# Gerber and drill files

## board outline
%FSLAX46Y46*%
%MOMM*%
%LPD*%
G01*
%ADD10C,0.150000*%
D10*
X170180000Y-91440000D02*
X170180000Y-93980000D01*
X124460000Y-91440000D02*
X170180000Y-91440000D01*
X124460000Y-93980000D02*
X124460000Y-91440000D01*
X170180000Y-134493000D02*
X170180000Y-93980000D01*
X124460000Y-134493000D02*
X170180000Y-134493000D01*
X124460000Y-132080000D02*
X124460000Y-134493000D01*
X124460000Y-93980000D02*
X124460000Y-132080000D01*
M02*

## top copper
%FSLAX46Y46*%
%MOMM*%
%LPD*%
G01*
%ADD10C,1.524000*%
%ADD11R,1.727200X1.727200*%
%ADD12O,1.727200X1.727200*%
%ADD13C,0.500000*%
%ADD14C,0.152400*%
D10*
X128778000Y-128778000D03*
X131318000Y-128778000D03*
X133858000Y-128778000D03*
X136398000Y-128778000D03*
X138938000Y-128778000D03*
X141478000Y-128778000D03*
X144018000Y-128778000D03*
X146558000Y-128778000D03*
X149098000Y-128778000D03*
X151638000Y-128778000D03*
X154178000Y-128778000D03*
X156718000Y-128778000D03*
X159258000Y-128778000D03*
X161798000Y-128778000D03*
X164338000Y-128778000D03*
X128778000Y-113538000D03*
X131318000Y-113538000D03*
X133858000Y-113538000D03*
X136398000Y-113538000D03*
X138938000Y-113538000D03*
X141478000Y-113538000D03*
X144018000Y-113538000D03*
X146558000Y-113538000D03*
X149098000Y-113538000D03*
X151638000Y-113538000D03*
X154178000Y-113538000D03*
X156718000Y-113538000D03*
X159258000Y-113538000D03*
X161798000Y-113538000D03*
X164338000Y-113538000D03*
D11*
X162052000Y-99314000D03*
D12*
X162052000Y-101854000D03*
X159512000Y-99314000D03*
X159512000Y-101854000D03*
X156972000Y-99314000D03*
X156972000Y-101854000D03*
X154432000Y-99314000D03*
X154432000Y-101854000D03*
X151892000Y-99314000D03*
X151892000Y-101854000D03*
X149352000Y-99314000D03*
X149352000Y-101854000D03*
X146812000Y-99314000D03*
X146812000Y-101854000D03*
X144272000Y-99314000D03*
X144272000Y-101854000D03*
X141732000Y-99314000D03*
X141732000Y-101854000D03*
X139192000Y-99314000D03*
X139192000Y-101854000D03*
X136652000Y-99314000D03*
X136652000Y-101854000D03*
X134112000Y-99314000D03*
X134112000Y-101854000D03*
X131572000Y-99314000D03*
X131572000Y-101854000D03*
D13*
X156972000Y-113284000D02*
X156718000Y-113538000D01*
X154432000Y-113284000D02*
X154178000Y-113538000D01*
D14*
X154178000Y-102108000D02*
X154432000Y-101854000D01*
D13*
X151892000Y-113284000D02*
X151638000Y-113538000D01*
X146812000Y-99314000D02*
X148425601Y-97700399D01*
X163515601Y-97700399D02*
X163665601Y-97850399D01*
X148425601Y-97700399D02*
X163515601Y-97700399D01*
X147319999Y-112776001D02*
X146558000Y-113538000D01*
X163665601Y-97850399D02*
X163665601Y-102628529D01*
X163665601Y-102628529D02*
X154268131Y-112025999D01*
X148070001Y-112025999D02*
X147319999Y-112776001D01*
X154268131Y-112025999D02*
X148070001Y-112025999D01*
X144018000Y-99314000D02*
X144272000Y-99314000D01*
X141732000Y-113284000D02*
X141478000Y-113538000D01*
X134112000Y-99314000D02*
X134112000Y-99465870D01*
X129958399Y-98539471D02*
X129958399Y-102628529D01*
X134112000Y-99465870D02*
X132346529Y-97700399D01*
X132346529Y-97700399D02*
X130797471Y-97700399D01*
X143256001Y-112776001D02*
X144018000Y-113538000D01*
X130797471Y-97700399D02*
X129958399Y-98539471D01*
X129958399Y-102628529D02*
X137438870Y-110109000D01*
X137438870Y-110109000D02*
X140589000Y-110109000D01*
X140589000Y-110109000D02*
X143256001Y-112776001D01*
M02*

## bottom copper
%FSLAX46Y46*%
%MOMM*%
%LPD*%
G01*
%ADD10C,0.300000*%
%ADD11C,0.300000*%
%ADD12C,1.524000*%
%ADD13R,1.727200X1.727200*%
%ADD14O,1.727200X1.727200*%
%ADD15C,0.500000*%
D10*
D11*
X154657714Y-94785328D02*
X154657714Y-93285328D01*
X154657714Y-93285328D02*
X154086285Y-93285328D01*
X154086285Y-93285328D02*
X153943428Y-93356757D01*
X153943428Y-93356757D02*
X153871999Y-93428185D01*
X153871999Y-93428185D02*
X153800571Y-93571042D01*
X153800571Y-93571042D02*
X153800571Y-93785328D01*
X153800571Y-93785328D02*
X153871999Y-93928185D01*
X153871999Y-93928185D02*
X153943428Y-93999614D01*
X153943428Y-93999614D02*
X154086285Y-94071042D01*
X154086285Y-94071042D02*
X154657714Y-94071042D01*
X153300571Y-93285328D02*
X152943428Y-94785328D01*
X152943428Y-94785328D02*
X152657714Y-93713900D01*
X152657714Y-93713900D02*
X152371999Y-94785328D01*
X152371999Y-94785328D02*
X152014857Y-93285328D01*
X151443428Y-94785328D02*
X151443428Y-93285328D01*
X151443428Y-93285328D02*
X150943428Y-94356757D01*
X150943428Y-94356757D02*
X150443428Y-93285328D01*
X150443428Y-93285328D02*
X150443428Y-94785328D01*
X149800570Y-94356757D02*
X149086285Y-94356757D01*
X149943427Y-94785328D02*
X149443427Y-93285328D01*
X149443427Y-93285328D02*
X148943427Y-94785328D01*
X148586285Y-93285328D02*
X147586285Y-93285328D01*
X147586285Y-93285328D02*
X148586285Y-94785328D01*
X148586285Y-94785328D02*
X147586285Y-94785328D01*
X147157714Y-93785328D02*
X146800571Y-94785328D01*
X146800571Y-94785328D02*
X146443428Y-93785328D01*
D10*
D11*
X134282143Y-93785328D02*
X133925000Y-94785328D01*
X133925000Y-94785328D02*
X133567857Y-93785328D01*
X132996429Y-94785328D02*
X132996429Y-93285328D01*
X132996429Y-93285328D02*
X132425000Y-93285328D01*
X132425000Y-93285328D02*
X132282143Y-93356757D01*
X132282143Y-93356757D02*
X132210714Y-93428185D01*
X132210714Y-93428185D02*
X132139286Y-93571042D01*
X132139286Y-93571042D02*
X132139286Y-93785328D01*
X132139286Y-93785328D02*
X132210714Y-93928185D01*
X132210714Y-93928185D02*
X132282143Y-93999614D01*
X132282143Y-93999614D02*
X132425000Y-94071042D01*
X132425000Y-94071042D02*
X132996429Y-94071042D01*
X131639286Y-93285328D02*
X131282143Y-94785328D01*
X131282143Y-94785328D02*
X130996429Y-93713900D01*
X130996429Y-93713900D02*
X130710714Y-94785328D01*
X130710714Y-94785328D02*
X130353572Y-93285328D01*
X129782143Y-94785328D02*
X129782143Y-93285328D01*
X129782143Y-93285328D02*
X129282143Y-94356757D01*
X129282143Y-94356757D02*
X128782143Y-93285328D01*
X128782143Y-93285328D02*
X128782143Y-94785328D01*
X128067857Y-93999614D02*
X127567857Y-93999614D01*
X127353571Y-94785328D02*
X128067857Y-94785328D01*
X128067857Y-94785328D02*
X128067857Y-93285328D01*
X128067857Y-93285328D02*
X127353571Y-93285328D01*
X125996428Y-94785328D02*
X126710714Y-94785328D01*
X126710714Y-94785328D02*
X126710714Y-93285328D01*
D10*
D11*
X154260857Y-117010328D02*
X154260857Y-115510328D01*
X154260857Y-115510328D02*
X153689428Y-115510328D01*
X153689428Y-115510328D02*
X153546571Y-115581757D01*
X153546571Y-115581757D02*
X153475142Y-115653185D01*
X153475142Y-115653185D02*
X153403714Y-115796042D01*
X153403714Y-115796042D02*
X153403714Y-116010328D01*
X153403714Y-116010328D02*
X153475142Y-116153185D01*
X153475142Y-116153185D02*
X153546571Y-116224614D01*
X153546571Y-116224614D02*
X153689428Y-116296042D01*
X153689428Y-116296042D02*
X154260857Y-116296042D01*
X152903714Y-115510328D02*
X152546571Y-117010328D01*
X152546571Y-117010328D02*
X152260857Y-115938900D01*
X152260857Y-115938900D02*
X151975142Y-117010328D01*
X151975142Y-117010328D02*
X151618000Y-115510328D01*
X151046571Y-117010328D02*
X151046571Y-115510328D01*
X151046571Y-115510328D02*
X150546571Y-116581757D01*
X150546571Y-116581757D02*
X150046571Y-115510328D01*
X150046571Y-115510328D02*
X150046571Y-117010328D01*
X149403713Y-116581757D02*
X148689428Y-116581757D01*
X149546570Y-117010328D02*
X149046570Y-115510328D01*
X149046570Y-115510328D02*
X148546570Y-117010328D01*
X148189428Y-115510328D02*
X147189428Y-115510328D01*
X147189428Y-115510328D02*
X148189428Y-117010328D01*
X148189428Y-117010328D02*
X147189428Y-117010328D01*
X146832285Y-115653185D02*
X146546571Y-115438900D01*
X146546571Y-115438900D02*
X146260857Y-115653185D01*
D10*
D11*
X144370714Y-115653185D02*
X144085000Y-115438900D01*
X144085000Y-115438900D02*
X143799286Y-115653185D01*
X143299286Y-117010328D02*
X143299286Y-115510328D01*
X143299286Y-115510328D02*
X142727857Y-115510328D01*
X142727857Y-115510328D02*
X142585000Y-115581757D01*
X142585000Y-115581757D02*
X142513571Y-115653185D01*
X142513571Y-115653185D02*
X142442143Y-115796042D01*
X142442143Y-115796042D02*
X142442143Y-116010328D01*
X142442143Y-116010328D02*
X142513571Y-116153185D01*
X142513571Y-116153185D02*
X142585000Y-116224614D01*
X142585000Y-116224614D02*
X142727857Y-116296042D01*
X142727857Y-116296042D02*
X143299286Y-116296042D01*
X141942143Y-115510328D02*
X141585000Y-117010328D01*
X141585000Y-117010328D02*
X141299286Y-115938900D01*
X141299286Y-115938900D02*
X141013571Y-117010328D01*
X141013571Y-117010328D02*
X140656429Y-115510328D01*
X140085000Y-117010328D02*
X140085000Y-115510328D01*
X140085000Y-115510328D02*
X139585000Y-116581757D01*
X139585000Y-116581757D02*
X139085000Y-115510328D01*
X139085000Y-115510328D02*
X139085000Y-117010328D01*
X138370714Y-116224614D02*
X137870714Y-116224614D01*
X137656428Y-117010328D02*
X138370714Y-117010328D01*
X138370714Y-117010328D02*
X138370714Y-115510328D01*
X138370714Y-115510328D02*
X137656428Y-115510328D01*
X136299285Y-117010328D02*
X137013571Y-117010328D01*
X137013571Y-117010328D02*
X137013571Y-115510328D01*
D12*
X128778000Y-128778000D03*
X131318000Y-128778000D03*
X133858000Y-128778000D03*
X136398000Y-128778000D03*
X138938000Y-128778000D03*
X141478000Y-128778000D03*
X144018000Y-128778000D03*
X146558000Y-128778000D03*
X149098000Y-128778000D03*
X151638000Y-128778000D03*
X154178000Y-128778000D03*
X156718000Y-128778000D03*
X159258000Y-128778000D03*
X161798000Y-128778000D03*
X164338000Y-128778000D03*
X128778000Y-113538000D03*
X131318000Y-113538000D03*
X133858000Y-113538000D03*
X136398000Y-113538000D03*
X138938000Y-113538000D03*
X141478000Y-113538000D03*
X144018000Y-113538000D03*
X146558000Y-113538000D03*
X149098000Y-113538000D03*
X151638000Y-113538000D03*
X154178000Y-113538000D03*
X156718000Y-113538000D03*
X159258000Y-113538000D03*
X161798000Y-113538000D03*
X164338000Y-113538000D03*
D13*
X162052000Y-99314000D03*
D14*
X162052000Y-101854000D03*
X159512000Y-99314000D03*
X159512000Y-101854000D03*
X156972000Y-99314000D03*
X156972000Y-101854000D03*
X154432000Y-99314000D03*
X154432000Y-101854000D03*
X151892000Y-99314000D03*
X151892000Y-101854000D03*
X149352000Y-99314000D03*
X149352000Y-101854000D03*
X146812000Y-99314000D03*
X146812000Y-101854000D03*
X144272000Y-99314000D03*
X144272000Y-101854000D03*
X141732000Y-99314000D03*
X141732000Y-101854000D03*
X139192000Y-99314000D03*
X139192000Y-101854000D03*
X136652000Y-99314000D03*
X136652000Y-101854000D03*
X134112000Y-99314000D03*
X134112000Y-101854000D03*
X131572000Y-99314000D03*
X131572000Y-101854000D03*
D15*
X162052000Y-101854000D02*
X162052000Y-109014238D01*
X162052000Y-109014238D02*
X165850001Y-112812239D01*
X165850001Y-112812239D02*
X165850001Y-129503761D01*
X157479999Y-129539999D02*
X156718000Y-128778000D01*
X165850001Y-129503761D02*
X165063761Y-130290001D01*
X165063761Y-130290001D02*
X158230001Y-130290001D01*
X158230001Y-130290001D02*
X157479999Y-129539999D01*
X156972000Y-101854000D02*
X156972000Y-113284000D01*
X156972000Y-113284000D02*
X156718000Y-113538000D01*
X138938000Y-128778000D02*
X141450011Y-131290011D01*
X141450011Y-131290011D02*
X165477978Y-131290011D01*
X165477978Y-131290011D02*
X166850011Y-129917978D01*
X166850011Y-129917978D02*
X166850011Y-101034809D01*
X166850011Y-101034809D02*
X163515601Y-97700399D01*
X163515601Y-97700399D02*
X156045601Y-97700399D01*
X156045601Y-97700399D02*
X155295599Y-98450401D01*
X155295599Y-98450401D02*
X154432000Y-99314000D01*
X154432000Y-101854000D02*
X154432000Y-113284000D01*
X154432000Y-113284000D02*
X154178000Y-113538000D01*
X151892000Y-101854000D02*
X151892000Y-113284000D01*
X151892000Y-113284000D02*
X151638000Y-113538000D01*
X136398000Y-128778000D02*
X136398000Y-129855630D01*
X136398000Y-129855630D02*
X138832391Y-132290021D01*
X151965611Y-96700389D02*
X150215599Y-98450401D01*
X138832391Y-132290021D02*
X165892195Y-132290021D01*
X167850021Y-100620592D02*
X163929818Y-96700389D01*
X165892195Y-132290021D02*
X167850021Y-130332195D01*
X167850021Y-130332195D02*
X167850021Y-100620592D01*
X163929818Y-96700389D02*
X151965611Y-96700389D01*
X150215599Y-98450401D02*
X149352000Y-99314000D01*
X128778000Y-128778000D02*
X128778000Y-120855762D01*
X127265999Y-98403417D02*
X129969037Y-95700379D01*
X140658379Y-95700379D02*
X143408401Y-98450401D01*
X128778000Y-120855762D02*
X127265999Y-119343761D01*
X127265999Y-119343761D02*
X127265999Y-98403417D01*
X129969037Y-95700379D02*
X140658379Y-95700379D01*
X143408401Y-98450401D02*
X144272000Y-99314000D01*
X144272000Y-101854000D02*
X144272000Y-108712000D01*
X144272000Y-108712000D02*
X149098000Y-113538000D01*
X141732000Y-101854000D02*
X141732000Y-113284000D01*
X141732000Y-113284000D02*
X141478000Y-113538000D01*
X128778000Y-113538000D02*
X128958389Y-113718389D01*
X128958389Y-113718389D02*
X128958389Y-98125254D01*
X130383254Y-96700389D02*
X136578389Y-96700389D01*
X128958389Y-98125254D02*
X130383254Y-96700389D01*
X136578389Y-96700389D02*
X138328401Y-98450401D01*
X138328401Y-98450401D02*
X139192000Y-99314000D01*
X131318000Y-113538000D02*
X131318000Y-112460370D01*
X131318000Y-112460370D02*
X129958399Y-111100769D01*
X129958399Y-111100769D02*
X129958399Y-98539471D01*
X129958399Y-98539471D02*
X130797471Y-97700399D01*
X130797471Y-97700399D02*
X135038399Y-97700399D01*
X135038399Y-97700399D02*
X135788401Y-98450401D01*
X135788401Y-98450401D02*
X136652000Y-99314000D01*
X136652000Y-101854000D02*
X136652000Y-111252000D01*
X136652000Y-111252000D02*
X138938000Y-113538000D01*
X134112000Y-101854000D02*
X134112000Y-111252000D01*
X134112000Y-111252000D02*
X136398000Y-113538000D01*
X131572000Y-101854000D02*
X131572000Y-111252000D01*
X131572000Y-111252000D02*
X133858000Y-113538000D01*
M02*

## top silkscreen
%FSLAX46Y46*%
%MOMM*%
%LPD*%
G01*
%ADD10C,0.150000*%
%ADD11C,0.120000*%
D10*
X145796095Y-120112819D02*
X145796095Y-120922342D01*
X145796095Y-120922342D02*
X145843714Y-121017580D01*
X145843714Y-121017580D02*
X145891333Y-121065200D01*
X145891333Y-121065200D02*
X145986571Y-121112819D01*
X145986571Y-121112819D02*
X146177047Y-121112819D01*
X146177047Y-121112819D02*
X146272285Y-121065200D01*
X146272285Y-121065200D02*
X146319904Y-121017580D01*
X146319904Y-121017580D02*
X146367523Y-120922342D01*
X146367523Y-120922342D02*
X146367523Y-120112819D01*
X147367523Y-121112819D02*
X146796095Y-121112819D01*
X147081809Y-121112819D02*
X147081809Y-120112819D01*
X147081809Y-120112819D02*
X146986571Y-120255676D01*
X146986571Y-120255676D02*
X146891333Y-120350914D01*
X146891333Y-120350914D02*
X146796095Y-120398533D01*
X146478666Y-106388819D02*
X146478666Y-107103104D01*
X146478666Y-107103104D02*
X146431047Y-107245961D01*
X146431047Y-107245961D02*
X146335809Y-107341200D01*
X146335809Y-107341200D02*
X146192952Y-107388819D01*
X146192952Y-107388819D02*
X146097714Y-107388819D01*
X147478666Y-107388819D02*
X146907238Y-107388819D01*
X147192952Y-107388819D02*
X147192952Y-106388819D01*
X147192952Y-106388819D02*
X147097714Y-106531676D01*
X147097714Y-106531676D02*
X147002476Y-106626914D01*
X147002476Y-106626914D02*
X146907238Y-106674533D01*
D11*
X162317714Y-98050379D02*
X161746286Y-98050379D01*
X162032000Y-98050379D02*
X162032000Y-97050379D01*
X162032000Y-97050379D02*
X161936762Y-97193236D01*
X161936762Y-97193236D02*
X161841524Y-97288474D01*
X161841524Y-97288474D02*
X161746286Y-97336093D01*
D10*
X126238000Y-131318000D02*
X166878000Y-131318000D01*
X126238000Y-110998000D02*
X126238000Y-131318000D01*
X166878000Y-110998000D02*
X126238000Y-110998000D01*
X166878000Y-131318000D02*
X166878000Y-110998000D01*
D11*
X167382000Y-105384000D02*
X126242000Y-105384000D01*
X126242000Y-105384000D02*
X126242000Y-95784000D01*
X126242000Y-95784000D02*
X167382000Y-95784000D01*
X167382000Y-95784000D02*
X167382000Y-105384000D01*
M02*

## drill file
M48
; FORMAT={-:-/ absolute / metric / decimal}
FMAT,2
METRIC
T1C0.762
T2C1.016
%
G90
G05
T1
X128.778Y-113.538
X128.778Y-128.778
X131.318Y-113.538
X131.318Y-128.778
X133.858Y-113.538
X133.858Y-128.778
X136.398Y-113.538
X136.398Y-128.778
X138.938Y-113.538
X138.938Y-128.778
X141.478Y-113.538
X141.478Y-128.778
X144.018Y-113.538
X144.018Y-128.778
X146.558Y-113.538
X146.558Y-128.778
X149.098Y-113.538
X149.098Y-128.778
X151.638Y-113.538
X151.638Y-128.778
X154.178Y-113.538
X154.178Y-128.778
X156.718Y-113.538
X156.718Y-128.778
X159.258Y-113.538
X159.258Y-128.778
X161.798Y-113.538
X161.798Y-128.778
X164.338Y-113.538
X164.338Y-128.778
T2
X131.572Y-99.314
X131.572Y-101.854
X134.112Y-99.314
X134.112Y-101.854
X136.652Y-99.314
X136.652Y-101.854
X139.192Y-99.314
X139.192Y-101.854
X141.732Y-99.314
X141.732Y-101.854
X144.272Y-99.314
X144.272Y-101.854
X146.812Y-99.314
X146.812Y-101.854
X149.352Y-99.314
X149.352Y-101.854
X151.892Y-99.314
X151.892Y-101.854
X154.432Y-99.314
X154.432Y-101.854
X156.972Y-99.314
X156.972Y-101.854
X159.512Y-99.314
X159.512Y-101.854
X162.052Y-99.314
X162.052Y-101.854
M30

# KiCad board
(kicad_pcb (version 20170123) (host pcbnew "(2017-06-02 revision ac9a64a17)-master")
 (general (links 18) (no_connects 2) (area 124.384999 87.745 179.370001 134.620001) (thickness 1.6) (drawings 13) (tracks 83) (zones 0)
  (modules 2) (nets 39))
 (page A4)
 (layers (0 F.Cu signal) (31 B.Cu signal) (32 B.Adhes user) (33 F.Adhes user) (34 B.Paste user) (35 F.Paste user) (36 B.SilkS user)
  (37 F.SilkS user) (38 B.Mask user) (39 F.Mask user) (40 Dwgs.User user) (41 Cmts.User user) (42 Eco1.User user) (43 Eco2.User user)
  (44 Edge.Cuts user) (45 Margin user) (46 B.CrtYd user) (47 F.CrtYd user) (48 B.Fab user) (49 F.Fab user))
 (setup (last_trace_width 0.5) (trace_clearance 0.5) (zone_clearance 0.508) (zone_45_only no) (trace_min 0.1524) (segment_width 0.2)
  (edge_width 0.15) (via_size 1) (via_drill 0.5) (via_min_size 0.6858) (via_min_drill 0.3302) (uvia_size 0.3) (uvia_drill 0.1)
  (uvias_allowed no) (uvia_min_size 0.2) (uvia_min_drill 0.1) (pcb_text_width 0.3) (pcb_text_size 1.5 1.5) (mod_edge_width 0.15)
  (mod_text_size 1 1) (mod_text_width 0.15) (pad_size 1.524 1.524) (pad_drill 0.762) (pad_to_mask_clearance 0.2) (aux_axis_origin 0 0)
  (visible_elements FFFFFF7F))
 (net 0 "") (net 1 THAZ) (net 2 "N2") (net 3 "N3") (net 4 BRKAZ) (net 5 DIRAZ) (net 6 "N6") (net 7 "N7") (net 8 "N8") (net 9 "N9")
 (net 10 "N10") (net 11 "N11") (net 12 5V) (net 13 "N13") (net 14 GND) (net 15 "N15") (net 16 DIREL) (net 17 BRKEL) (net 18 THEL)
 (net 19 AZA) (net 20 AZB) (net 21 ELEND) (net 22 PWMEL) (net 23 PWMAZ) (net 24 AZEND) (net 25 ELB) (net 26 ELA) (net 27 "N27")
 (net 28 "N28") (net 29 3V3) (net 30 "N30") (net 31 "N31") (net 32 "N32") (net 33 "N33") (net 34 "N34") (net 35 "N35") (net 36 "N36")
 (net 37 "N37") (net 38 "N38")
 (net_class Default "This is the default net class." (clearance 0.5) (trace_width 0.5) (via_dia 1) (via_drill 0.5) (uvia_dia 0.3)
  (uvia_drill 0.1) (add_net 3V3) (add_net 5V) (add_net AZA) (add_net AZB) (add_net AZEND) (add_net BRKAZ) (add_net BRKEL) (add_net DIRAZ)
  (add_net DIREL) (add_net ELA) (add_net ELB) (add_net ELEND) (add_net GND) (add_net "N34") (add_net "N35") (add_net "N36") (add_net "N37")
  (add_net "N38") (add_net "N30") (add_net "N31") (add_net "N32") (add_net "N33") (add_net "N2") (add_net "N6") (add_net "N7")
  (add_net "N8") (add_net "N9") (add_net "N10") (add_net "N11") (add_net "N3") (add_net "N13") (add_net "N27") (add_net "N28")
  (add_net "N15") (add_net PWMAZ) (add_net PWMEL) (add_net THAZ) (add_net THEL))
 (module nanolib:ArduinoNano (layer F.Cu) (at 146.558 121.158 180)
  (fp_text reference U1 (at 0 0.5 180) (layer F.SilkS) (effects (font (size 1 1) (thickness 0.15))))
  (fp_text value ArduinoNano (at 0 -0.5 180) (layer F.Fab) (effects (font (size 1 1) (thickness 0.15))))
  (fp_line (start 20.32 -10.16) (end -20.32 -10.16) (layer F.SilkS) (width 0.15))
  (fp_line (start 20.32 10.16) (end 20.32 -10.16) (layer F.SilkS) (width 0.15))
  (fp_line (start -20.32 10.16) (end 20.32 10.16) (layer F.SilkS) (width 0.15))
  (fp_line (start -20.32 -10.16) (end -20.32 10.16) (layer F.SilkS) (width 0.15))
  (pad D13 thru_hole circle (at 17.78 -7.62 180) (size 1.524 1.524) (drill 0.762) (layers *.Cu *.Mask) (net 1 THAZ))
  (pad 3V3 thru_hole circle (at 15.24 -7.62 180) (size 1.524 1.524) (drill 0.762) (layers *.Cu *.Mask) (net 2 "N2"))
  (pad REF thru_hole circle (at 12.7 -7.62 180) (size 1.524 1.524) (drill 0.762) (layers *.Cu *.Mask) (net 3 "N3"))
  (pad A0 thru_hole circle (at 10.16 -7.62 180) (size 1.524 1.524) (drill 0.762) (layers *.Cu *.Mask) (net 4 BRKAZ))
  (pad A1 thru_hole circle (at 7.62 -7.62 180) (size 1.524 1.524) (drill 0.762) (layers *.Cu *.Mask) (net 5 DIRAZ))
  (pad A2 thru_hole circle (at 5.08 -7.62 180) (size 1.524 1.524) (drill 0.762) (layers *.Cu *.Mask) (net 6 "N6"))
  (pad A3 thru_hole circle (at 2.54 -7.62 180) (size 1.524 1.524) (drill 0.762) (layers *.Cu *.Mask) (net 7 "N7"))
  (pad A4 thru_hole circle (at 0 -7.62 180) (size 1.524 1.524) (drill 0.762) (layers *.Cu *.Mask) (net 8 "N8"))
  (pad A5 thru_hole circle (at -2.54 -7.62 180) (size 1.524 1.524) (drill 0.762) (layers *.Cu *.Mask) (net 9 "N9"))
  (pad A6 thru_hole circle (at -5.08 -7.62 180) (size 1.524 1.524) (drill 0.762) (layers *.Cu *.Mask) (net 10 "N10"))
  (pad A7 thru_hole circle (at -7.62 -7.62 180) (size 1.524 1.524) (drill 0.762) (layers *.Cu *.Mask) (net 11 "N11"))
  (pad 5V thru_hole circle (at -10.16 -7.62 180) (size 1.524 1.524) (drill 0.762) (layers *.Cu *.Mask) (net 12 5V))
  (pad RST thru_hole circle (at -12.7 -7.62 180) (size 1.524 1.524) (drill 0.762) (layers *.Cu *.Mask) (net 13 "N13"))
  (pad GND thru_hole circle (at -15.24 -7.62 180) (size 1.524 1.524) (drill 0.762) (layers *.Cu *.Mask) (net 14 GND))
  (pad VIN thru_hole circle (at -17.78 -7.62 180) (size 1.524 1.524) (drill 0.762) (layers *.Cu *.Mask) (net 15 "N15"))
  (pad D12 thru_hole circle (at 17.78 7.62 180) (size 1.524 1.524) (drill 0.762) (layers *.Cu *.Mask) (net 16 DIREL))
  (pad D11 thru_hole circle (at 15.24 7.62 180) (size 1.524 1.524) (drill 0.762) (layers *.Cu *.Mask) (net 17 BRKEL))
  (pad D10 thru_hole circle (at 12.7 7.62 180) (size 1.524 1.524) (drill 0.762) (layers *.Cu *.Mask) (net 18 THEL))
  (pad D9 thru_hole circle (at 10.16 7.62 180) (size 1.524 1.524) (drill 0.762) (layers *.Cu *.Mask) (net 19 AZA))
  (pad D8 thru_hole circle (at 7.62 7.62 180) (size 1.524 1.524) (drill 0.762) (layers *.Cu *.Mask) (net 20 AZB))
  (pad D7 thru_hole circle (at 5.08 7.62 180) (size 1.524 1.524) (drill 0.762) (layers *.Cu *.Mask) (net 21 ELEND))
  (pad D6 thru_hole circle (at 2.54 7.62 180) (size 1.524 1.524) (drill 0.762) (layers *.Cu *.Mask) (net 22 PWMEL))
  (pad D5 thru_hole circle (at 0 7.62 180) (size 1.524 1.524) (drill 0.762) (layers *.Cu *.Mask) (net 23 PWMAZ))
  (pad D4 thru_hole circle (at -2.54 7.62 180) (size 1.524 1.524) (drill 0.762) (layers *.Cu *.Mask) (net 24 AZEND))
  (pad D3 thru_hole circle (at -5.08 7.62 180) (size 1.524 1.524) (drill 0.762) (layers *.Cu *.Mask) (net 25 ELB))
  (pad D2 thru_hole circle (at -7.62 7.62 180) (size 1.524 1.524) (drill 0.762) (layers *.Cu *.Mask) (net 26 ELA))
  (pad GND thru_hole circle (at -10.16 7.62 180) (size 1.524 1.524) (drill 0.762) (layers *.Cu *.Mask) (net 14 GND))
  (pad RST thru_hole circle (at -12.7 7.62 180) (size 1.524 1.524) (drill 0.762) (layers *.Cu *.Mask) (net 13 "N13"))
  (pad RX0 thru_hole circle (at -15.24 7.62 180) (size 1.524 1.524) (drill 0.762) (layers *.Cu *.Mask) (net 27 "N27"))
  (pad TX1 thru_hole circle (at -17.78 7.62 180) (size 1.524 1.524) (drill 0.762) (layers *.Cu *.Mask) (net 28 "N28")))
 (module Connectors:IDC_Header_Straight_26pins (layer F.Cu) (at 162.052 99.314 180)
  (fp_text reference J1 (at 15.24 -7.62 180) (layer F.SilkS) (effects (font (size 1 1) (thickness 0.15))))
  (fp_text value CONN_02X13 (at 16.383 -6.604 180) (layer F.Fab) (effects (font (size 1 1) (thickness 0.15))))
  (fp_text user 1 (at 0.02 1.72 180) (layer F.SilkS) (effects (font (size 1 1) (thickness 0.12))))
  (fp_line (start -5.33 -6.07) (end 35.81 -6.07) (layer F.SilkS) (width 0.12))
  (fp_line (start 35.81 -6.07) (end 35.81 3.53) (layer F.SilkS) (width 0.12))
  (fp_line (start 35.81 3.53) (end -5.33 3.53) (layer F.SilkS) (width 0.12))
  (fp_line (start -5.33 3.53) (end -5.33 -6.07) (layer F.SilkS) (width 0.12))
  (pad 1 thru_hole rect (at 0 0 180) (size 1.7272 1.7272) (drill 1.016) (layers *.Cu *.Mask) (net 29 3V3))
  (pad 2 thru_hole oval (at 0 -2.54 180) (size 1.7272 1.7272) (drill 1.016) (layers *.Cu *.Mask) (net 12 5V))
  (pad 3 thru_hole oval (at 2.54 0 180) (size 1.7272 1.7272) (drill 1.016) (layers *.Cu *.Mask) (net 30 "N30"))
  (pad 4 thru_hole oval (at 2.54 -2.54 180) (size 1.7272 1.7272) (drill 1.016) (layers *.Cu *.Mask) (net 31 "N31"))
  (pad 5 thru_hole oval (at 5.08 0 180) (size 1.7272 1.7272) (drill 1.016) (layers *.Cu *.Mask) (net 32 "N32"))
  (pad 6 thru_hole oval (at 5.08 -2.54 180) (size 1.7272 1.7272) (drill 1.016) (layers *.Cu *.Mask) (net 14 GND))
  (pad 7 thru_hole oval (at 7.62 0 180) (size 1.7272 1.7272) (drill 1.016) (layers *.Cu *.Mask) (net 5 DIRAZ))
  (pad 8 thru_hole oval (at 7.62 -2.54 180) (size 1.7272 1.7272) (drill 1.016) (layers *.Cu *.Mask) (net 26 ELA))
  (pad 9 thru_hole oval (at 10.16 0 180) (size 1.7272 1.7272) (drill 1.016) (layers *.Cu *.Mask) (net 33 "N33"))
  (pad 10 thru_hole oval (at 10.16 -2.54 180) (size 1.7272 1.7272) (drill 1.016) (layers *.Cu *.Mask) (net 25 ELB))
  (pad 11 thru_hole oval (at 12.7 0 180) (size 1.7272 1.7272) (drill 1.016) (layers *.Cu *.Mask) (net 4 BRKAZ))
  (pad 12 thru_hole oval (at 12.7 -2.54 180) (size 1.7272 1.7272) (drill 1.016) (layers *.Cu *.Mask) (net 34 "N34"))
  (pad 13 thru_hole oval (at 15.24 0 180) (size 1.7272 1.7272) (drill 1.016) (layers *.Cu *.Mask) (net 23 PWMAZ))
  (pad 14 thru_hole oval (at 15.24 -2.54 180) (size 1.7272 1.7272) (drill 1.016) (layers *.Cu *.Mask) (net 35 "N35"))
  (pad 15 thru_hole oval (at 17.78 0 180) (size 1.7272 1.7272) (drill 1.016) (layers *.Cu *.Mask) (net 1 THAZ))
  (pad 16 thru_hole oval (at 17.78 -2.54 180) (size 1.7272 1.7272) (drill 1.016) (layers *.Cu *.Mask) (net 24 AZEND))
  (pad 17 thru_hole oval (at 20.32 0 180) (size 1.7272 1.7272) (drill 1.016) (layers *.Cu *.Mask) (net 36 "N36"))
  (pad 18 thru_hole oval (at 20.32 -2.54 180) (size 1.7272 1.7272) (drill 1.016) (layers *.Cu *.Mask) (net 21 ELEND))
  (pad 19 thru_hole oval (at 22.86 0 180) (size 1.7272 1.7272) (drill 1.016) (layers *.Cu *.Mask) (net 16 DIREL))
  (pad 20 thru_hole oval (at 22.86 -2.54 180) (size 1.7272 1.7272) (drill 1.016) (layers *.Cu *.Mask) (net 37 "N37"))
  (pad 21 thru_hole oval (at 25.4 0 180) (size 1.7272 1.7272) (drill 1.016) (layers *.Cu *.Mask) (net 17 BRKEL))
  (pad 22 thru_hole oval (at 25.4 -2.54 180) (size 1.7272 1.7272) (drill 1.016) (layers *.Cu *.Mask) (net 20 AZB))
  (pad 23 thru_hole oval (at 27.94 0 180) (size 1.7272 1.7272) (drill 1.016) (layers *.Cu *.Mask) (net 22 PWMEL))
  (pad 24 thru_hole oval (at 27.94 -2.54 180) (size 1.7272 1.7272) (drill 1.016) (layers *.Cu *.Mask) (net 19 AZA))
  (pad 25 thru_hole oval (at 30.48 0 180) (size 1.7272 1.7272) (drill 1.016) (layers *.Cu *.Mask) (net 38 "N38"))
  (pad 26 thru_hole oval (at 30.48 -2.54 180) (size 1.7272 1.7272) (drill 1.016) (layers *.Cu *.Mask) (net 18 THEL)))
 (gr_line (start 170.18 91.44) (end 170.18 93.98) (layer Edge.Cuts) (width 0.15))
 (gr_line (start 124.46 91.44) (end 170.18 91.44) (layer Edge.Cuts) (width 0.15))
 (gr_line (start 124.46 93.98) (end 124.46 91.44) (layer Edge.Cuts) (width 0.15))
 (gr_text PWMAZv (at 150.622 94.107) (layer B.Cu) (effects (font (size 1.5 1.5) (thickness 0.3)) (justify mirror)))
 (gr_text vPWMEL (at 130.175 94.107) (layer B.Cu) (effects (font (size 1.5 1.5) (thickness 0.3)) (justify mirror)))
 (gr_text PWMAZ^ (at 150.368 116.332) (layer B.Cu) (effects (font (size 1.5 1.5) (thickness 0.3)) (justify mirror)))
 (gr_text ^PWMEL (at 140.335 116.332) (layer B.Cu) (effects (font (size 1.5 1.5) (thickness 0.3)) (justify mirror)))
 (gr_line (start 170.18 134.493) (end 170.18 93.98) (layer Edge.Cuts) (width 0.15))
 (gr_line (start 124.46 134.493) (end 170.18 134.493) (layer Edge.Cuts) (width 0.15))
 (gr_line (start 124.46 132.08) (end 124.46 134.493) (layer Edge.Cuts) (width 0.15))
 (gr_line (start 124.46 93.98) (end 124.46 132.08) (layer Edge.Cuts) (width 0.15))
 (segment (start 162.052 101.854) (end 162.052 109.014238) (width 0.5) (layer B.Cu) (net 12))
 (segment (start 162.052 109.014238) (end 165.850001 112.812239) (width 0.5) (layer B.Cu) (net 12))
 (segment (start 165.850001 112.812239) (end 165.850001 129.503761) (width 0.5) (layer B.Cu) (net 12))
 (segment (start 157.479999 129.539999) (end 156.718 128.778) (width 0.5) (layer B.Cu) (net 12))
 (segment (start 165.850001 129.503761) (end 165.063761 130.290001) (width 0.5) (layer B.Cu) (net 12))
 (segment (start 165.063761 130.290001) (end 158.230001 130.290001) (width 0.5) (layer B.Cu) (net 12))
 (segment (start 158.230001 130.290001) (end 157.479999 129.539999) (width 0.5) (layer B.Cu) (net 12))
 (segment (start 156.972 101.854) (end 156.972 113.284) (width 0.5) (layer B.Cu) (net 14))
 (segment (start 156.972 113.284) (end 156.718 113.538) (width 0.5) (layer B.Cu) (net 14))
 (segment (start 156.972 113.284) (end 156.718 113.538) (width 0.5) (layer F.Cu) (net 14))
 (segment (start 138.938 128.778) (end 141.450011 131.290011) (width 0.5) (layer B.Cu) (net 5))
 (segment (start 141.450011 131.290011) (end 165.477978 131.290011) (width 0.5) (layer B.Cu) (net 5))
 (segment (start 165.477978 131.290011) (end 166.850011 129.917978) (width 0.5) (layer B.Cu) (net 5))
 (segment (start 166.850011 129.917978) (end 166.850011 101.034809) (width 0.5) (layer B.Cu) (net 5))
 (segment (start 166.850011 101.034809) (end 163.515601 97.700399) (width 0.5) (layer B.Cu) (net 5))
 (segment (start 163.515601 97.700399) (end 156.045601 97.700399) (width 0.5) (layer B.Cu) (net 5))
 (segment (start 156.045601 97.700399) (end 155.295599 98.450401) (width 0.5) (layer B.Cu) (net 5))
 (segment (start 155.295599 98.450401) (end 154.432 99.314) (width 0.5) (layer B.Cu) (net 5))
 (segment (start 154.432 101.854) (end 154.432 113.284) (width 0.5) (layer B.Cu) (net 26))
 (segment (start 154.432 113.284) (end 154.178 113.538) (width 0.5) (layer B.Cu) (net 26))
 (segment (start 154.432 113.284) (end 154.178 113.538) (width 0.5) (layer F.Cu) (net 26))
 (segment (start 154.178 102.108) (end 154.432 101.854) (width 0.1524) (layer F.Cu) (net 26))
 (segment (start 151.892 101.854) (end 151.892 113.284) (width 0.5) (layer B.Cu) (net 25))
 (segment (start 151.892 113.284) (end 151.638 113.538) (width 0.5) (layer B.Cu) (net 25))
 (segment (start 151.892 113.284) (end 151.638 113.538) (width 0.5) (layer F.Cu) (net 25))
 (segment (start 136.398 128.778) (end 136.398 129.85563) (width 0.5) (layer B.Cu) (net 4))
 (segment (start 136.398 129.85563) (end 138.832391 132.290021) (width 0.5) (layer B.Cu) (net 4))
 (segment (start 151.965611 96.700389) (end 150.215599 98.450401) (width 0.5) (layer B.Cu) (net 4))
 (segment (start 138.832391 132.290021) (end 165.892195 132.290021) (width 0.5) (layer B.Cu) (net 4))
 (segment (start 167.850021 100.620592) (end 163.929818 96.700389) (width 0.5) (layer B.Cu) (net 4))
 (segment (start 165.892195 132.290021) (end 167.850021 130.332195) (width 0.5) (layer B.Cu) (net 4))
 (segment (start 167.850021 130.332195) (end 167.850021 100.620592) (width 0.5) (layer B.Cu) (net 4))
 (segment (start 163.929818 96.700389) (end 151.965611 96.700389) (width 0.5) (layer B.Cu) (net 4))
 (segment (start 150.215599 98.450401) (end 149.352 99.314) (width 0.5) (layer B.Cu) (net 4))
 (segment (start 146.812 99.314) (end 148.425601 97.700399) (width 0.5) (layer F.Cu) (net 23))
 (segment (start 163.515601 97.700399) (end 163.665601 97.850399) (width 0.5) (layer F.Cu) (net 23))
 (segment (start 148.425601 97.700399) (end 163.515601 97.700399) (width 0.5) (layer F.Cu) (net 23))
 (segment (start 147.319999 112.776001) (end 146.558 113.538) (width 0.5) (layer F.Cu) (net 23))
 (segment (start 163.665601 97.850399) (end 163.665601 102.628529) (width 0.5) (layer F.Cu) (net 23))
 (segment (start 163.665601 102.628529) (end 154.268131 112.025999) (width 0.5) (layer F.Cu) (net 23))
 (segment (start 148.070001 112.025999) (end 147.319999 112.776001) (width 0.5) (layer F.Cu) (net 23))
 (segment (start 154.268131 112.025999) (end 148.070001 112.025999) (width 0.5) (layer F.Cu) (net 23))
 (segment (start 128.778 128.778) (end 128.778 120.855762) (width 0.5) (layer B.Cu) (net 1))
 (segment (start 127.265999 98.403417) (end 129.969037 95.700379) (width 0.5) (layer B.Cu) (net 1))
 (segment (start 140.658379 95.700379) (end 143.408401 98.450401) (width 0.5) (layer B.Cu) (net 1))
 (segment (start 128.778 120.855762) (end 127.265999 119.343761) (width 0.5) (layer B.Cu) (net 1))
 (segment (start 127.265999 119.343761) (end 127.265999 98.403417) (width 0.5) (layer B.Cu) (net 1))
 (segment (start 129.969037 95.700379) (end 140.658379 95.700379) (width 0.5) (layer B.Cu) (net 1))
 (segment (start 143.408401 98.450401) (end 144.272 99.314) (width 0.5) (layer B.Cu) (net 1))
 (segment (start 144.018 99.314) (end 144.272 99.314) (width 0.5) (layer F.Cu) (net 1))
 (segment (start 144.272 101.854) (end 144.272 108.712) (width 0.5) (layer B.Cu) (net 24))
 (segment (start 144.272 108.712) (end 149.098 113.538) (width 0.5) (layer B.Cu) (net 24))
 (segment (start 141.732 101.854) (end 141.732 113.284) (width 0.5) (layer B.Cu) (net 21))
 (segment (start 141.732 113.284) (end 141.478 113.538) (width 0.5) (layer B.Cu) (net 21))
 (segment (start 141.732 113.284) (end 141.478 113.538) (width 0.5) (layer F.Cu) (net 21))
 (segment (start 128.778 113.538) (end 128.958389 113.718389) (width 0.5) (layer B.Cu) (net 16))
 (segment (start 128.958389 113.718389) (end 128.958389 98.125254) (width 0.5) (layer B.Cu) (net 16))
 (segment (start 130.383254 96.700389) (end 136.578389 96.700389) (width 0.5) (layer B.Cu) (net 16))
 (segment (start 128.958389 98.125254) (end 130.383254 96.700389) (width 0.5) (layer B.Cu) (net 16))
 (segment (start 136.578389 96.700389) (end 138.328401 98.450401) (width 0.5) (layer B.Cu) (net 16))
 (segment (start 138.328401 98.450401) (end 139.192 99.314) (width 0.5) (layer B.Cu) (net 16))
 (segment (start 131.318 113.538) (end 131.318 112.46037) (width 0.5) (layer B.Cu) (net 17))
 (segment (start 131.318 112.46037) (end 129.958399 111.100769) (width 0.5) (layer B.Cu) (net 17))
 (segment (start 129.958399 111.100769) (end 129.958399 98.539471) (width 0.5) (layer B.Cu) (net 17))
 (segment (start 129.958399 98.539471) (end 130.797471 97.700399) (width 0.5) (layer B.Cu) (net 17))
 (segment (start 130.797471 97.700399) (end 135.038399 97.700399) (width 0.5) (layer B.Cu) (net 17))
 (segment (start 135.038399 97.700399) (end 135.788401 98.450401) (width 0.5) (layer B.Cu) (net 17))
 (segment (start 135.788401 98.450401) (end 136.652 99.314) (width 0.5) (layer B.Cu) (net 17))
 (segment (start 136.652 101.854) (end 136.652 111.252) (width 0.5) (layer B.Cu) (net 20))
 (segment (start 136.652 111.252) (end 138.938 113.538) (width 0.5) (layer B.Cu) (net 20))
 (segment (start 134.112 99.314) (end 134.112 99.46587) (width 0.5) (layer F.Cu) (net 22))
 (segment (start 129.958399 98.539471) (end 129.958399 102.628529) (width 0.5) (layer F.Cu) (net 22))
 (segment (start 134.112 99.46587) (end 132.346529 97.700399) (width 0.5) (layer F.Cu) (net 22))
 (segment (start 132.346529 97.700399) (end 130.797471 97.700399) (width 0.5) (layer F.Cu) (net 22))
 (segment (start 143.256001 112.776001) (end 144.018 113.538) (width 0.5) (layer F.Cu) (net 22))
 (segment (start 130.797471 97.700399) (end 129.958399 98.539471) (width 0.5) (layer F.Cu) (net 22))
 (segment (start 129.958399 102.628529) (end 137.43887 110.109) (width 0.5) (layer F.Cu) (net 22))
 (segment (start 137.43887 110.109) (end 140.589 110.109) (width 0.5) (layer F.Cu) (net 22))
 (segment (start 140.589 110.109) (end 143.256001 112.776001) (width 0.5) (layer F.Cu) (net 22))
 (segment (start 134.112 101.854) (end 134.112 111.252) (width 0.5) (layer B.Cu) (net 19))
 (segment (start 134.112 111.252) (end 136.398 113.538) (width 0.5) (layer B.Cu) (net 19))
 (segment (start 131.572 101.854) (end 131.572 111.252) (width 0.5) (layer B.Cu) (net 18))
 (segment (start 131.572 111.252) (end 133.858 113.538) (width 0.5) (layer B.Cu) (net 18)))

